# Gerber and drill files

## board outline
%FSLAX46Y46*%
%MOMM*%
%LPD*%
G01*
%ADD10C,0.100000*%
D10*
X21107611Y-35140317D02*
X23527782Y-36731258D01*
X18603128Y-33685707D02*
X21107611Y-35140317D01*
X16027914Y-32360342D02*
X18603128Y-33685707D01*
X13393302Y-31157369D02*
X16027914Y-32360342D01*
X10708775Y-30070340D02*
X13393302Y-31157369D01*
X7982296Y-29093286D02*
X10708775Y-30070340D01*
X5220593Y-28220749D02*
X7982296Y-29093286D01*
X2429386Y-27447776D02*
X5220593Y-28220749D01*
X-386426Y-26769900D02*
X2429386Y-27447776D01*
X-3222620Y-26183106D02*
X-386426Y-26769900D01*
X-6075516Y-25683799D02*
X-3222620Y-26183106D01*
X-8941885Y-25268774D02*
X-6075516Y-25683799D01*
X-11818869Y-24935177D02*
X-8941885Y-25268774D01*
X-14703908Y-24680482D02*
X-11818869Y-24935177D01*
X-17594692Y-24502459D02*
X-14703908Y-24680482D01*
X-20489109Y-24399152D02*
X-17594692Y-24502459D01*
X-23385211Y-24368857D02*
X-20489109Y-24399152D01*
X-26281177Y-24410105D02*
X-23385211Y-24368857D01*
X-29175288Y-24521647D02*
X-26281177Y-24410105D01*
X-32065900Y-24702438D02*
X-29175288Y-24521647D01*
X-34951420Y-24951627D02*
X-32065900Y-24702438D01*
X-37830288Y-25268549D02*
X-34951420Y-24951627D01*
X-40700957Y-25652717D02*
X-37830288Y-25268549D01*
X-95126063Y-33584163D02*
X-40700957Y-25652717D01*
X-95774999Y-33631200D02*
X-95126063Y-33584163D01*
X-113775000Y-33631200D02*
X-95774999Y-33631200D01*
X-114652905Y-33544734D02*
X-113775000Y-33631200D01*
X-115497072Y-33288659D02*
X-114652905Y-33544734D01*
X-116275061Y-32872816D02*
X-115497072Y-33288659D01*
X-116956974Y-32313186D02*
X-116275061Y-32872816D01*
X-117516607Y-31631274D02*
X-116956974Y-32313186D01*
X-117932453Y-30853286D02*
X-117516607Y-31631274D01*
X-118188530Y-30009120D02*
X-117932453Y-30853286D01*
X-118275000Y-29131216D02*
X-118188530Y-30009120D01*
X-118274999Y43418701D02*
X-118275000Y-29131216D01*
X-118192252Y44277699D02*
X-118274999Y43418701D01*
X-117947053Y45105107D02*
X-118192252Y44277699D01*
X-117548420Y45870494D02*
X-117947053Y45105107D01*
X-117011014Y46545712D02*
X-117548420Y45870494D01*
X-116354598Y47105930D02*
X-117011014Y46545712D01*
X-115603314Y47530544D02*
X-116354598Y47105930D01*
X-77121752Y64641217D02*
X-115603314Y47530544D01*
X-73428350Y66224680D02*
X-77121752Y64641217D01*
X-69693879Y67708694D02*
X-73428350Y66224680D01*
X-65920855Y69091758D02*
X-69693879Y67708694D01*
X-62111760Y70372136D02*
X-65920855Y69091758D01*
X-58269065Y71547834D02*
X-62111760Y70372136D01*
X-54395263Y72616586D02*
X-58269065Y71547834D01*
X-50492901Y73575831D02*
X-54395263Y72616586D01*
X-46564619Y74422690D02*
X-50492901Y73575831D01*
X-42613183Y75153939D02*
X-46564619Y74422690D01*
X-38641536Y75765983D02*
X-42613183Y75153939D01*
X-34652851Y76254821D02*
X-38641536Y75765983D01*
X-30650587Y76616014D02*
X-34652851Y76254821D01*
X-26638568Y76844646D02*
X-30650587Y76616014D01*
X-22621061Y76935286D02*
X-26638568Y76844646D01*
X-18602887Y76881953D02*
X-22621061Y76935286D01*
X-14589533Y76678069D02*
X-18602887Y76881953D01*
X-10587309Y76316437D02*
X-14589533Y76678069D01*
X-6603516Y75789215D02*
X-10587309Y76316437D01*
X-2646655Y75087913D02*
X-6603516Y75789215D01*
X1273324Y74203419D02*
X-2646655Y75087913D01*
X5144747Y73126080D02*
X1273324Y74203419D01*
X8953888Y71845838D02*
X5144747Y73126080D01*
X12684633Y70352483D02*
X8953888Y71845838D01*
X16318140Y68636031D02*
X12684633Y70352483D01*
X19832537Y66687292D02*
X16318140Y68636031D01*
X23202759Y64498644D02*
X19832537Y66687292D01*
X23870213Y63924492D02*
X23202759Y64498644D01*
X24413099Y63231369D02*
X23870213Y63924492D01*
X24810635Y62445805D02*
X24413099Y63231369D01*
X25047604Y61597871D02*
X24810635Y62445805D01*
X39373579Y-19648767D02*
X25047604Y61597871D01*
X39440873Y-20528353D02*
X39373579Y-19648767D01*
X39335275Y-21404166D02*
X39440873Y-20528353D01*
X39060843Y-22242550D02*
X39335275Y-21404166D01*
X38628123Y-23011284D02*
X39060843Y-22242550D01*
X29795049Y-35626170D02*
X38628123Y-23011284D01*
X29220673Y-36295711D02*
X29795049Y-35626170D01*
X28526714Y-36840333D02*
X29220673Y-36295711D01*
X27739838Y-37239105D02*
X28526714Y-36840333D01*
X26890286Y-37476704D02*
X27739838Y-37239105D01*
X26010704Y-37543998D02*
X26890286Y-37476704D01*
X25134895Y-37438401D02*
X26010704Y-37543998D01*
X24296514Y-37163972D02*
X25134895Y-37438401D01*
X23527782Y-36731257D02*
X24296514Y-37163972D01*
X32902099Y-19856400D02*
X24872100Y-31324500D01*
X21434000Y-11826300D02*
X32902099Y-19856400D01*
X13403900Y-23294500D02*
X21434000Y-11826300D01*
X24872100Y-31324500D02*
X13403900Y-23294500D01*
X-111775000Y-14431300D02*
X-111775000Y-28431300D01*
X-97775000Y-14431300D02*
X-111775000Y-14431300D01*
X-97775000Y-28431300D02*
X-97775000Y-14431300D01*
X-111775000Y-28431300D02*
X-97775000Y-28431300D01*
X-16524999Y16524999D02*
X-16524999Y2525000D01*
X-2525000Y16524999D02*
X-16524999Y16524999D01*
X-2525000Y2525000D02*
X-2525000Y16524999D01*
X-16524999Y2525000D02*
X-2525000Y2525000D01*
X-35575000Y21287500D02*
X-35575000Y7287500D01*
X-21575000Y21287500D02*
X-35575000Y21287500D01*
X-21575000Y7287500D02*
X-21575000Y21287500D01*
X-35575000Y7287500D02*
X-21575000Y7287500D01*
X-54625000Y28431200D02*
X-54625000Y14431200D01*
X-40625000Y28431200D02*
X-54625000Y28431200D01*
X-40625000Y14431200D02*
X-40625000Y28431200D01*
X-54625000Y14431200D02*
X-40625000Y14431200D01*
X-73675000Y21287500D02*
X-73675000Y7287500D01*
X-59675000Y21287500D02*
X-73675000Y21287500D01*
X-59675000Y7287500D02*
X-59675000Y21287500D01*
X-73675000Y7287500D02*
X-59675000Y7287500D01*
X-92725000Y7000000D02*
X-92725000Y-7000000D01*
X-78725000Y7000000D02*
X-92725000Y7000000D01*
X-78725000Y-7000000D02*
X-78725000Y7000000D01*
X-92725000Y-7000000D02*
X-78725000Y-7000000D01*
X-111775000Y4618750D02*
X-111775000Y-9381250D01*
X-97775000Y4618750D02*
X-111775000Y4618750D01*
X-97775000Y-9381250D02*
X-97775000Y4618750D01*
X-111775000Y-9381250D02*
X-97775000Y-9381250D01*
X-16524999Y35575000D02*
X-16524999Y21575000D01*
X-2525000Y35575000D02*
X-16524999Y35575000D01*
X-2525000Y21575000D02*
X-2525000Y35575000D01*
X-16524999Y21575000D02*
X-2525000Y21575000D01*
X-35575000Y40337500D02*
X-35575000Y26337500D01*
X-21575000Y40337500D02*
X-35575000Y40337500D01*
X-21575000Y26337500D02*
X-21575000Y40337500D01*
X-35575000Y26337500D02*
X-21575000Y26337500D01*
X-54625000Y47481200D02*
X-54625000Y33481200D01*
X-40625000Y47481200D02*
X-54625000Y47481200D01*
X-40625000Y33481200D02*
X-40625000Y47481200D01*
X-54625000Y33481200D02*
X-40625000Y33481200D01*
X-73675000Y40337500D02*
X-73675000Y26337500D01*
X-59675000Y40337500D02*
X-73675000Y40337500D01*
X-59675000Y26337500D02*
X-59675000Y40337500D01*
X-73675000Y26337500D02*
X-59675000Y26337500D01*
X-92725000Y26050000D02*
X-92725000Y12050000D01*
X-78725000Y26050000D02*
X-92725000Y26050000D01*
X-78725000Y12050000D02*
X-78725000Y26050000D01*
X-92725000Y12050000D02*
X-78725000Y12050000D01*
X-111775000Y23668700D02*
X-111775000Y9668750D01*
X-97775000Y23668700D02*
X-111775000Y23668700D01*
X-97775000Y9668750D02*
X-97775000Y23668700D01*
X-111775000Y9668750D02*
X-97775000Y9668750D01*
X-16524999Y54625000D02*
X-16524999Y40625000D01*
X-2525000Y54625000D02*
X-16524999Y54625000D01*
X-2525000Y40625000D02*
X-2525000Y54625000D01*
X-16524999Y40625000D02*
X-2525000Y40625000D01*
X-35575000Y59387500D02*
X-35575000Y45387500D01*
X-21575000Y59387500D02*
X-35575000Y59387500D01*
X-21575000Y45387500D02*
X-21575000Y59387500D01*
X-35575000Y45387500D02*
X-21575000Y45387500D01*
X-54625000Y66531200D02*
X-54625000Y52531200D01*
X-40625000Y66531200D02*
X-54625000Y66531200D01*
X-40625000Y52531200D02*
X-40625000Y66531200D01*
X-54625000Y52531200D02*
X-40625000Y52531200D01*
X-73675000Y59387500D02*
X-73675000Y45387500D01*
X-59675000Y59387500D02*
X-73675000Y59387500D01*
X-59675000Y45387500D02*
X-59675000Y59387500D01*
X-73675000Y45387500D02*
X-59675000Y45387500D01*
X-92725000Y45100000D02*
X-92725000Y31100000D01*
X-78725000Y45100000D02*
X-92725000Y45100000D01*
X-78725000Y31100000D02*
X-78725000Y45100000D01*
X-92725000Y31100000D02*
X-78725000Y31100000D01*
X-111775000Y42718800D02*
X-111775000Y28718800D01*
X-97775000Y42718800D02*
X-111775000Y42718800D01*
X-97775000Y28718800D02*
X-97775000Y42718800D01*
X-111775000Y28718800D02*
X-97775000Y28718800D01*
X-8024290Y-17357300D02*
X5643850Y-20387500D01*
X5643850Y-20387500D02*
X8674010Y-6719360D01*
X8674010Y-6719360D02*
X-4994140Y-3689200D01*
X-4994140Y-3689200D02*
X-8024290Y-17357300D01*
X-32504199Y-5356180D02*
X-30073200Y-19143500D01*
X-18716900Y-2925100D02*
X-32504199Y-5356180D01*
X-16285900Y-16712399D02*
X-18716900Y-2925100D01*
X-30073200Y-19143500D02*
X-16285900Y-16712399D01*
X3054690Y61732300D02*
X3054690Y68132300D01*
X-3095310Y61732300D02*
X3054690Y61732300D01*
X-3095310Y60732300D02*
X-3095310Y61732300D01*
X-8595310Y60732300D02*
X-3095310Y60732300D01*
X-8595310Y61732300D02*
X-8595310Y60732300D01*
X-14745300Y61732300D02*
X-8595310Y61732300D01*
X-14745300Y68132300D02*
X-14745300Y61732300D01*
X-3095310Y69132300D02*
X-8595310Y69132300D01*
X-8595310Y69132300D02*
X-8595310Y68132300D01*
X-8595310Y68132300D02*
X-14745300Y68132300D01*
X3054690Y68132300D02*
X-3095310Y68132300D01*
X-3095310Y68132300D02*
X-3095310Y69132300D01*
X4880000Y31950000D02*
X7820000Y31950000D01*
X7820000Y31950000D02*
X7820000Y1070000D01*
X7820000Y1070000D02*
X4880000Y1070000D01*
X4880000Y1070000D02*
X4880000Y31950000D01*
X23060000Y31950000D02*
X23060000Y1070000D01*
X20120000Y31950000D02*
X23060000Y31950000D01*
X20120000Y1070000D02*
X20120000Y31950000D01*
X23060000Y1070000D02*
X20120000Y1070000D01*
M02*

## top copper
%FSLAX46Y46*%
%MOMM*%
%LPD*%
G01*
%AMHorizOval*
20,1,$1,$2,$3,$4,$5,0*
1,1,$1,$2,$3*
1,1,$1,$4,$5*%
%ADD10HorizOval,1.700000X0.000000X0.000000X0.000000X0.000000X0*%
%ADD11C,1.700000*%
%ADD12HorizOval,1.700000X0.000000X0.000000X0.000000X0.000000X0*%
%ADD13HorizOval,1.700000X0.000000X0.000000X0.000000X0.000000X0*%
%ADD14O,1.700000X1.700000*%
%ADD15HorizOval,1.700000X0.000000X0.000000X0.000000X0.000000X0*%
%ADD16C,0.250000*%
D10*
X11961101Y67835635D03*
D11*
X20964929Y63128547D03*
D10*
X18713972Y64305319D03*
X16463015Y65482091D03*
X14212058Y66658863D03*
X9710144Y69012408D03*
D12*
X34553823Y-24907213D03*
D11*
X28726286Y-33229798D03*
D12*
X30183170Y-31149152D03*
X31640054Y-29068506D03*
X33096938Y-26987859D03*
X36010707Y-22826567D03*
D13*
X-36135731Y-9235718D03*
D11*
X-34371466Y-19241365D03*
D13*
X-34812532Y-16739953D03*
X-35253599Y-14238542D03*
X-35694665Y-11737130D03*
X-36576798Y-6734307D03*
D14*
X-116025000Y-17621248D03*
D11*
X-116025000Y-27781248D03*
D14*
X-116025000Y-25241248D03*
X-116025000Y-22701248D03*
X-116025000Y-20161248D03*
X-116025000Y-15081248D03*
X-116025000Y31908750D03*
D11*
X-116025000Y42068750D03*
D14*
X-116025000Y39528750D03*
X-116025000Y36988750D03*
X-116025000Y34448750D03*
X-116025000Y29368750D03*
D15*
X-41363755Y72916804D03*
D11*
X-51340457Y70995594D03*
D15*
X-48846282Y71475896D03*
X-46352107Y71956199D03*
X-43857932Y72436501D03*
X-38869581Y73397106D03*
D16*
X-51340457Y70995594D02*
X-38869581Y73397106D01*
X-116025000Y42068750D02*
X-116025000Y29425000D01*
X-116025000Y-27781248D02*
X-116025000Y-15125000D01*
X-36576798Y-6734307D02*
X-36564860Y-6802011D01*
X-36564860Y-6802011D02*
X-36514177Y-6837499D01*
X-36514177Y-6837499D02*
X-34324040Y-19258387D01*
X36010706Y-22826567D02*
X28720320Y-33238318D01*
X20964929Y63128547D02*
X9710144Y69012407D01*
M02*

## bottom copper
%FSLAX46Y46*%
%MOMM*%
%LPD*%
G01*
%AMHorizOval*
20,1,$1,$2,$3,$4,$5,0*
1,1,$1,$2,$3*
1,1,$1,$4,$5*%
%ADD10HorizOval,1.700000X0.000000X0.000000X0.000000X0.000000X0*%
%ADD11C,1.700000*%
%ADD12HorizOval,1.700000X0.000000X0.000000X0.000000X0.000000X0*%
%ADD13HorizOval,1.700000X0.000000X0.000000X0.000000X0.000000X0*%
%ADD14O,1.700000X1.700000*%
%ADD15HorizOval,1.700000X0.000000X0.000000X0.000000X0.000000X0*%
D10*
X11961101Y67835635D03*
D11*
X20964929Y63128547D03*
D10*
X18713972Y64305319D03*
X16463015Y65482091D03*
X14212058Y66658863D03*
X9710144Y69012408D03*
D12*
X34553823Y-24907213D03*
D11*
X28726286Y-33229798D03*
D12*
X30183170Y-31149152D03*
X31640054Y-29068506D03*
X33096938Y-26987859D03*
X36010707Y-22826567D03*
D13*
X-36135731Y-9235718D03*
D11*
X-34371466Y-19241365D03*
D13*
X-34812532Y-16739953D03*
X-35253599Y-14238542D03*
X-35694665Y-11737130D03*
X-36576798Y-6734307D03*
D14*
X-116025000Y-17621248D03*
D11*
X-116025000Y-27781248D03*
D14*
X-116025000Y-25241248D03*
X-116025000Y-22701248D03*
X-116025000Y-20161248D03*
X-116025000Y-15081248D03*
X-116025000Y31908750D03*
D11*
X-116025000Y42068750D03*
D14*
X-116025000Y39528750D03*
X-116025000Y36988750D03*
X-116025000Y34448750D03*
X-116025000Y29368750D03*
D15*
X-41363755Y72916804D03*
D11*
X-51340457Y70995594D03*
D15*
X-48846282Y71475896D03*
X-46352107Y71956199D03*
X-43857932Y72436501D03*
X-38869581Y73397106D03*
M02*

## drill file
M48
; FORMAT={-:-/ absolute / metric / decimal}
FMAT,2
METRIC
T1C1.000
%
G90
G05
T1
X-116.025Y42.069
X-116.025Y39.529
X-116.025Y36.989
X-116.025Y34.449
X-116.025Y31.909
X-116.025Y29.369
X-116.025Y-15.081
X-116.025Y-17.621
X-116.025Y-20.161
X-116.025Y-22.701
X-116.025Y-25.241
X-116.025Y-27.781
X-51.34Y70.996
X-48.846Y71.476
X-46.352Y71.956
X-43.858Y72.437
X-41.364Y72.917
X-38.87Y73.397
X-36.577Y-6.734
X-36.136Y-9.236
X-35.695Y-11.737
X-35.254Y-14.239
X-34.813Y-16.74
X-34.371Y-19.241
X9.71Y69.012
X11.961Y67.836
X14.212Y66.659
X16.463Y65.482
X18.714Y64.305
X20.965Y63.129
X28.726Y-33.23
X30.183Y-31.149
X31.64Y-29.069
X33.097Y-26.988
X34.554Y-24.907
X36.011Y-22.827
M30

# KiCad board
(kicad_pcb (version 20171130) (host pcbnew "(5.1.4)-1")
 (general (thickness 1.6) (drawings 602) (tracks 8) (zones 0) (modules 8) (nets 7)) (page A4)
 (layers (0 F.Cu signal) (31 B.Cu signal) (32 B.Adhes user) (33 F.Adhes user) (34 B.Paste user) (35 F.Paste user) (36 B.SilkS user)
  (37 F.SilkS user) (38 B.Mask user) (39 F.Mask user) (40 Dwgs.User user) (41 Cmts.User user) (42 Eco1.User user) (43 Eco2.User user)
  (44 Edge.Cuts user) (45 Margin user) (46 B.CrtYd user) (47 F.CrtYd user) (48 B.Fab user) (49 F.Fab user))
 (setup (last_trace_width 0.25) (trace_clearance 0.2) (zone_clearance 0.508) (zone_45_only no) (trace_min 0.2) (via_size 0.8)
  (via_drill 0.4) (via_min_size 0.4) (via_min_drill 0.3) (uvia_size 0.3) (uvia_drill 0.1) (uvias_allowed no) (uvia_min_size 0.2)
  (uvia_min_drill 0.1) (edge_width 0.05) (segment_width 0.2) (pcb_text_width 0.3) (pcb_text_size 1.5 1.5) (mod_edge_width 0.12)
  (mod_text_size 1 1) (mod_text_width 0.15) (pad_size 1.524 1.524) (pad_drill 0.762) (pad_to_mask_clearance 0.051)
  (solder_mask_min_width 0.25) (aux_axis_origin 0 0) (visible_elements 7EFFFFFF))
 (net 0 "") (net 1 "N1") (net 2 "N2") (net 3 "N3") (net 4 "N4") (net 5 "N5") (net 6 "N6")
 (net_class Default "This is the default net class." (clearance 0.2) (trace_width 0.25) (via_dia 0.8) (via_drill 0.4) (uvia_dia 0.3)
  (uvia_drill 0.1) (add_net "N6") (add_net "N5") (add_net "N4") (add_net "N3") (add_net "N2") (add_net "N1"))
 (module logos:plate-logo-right (layer B.Cu) (at 13.97 -26.2255 180)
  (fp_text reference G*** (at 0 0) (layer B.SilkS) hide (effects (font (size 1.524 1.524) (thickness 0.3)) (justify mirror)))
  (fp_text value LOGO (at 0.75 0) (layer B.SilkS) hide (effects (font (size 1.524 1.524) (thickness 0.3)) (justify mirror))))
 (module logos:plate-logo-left (layer F.Cu) (at 13.97 -26.2255)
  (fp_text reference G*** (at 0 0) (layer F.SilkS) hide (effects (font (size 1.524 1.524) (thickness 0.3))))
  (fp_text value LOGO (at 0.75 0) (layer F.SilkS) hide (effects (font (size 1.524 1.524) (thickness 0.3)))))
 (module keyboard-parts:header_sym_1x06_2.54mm (layer F.Cu) (at 20.964929 -63.128547 242.4)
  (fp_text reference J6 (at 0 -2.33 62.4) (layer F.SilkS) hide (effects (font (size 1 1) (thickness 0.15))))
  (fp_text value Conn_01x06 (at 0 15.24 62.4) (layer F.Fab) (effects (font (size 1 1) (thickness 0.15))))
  (pad 5 thru_hole oval (at 0 10.16 242.4) (size 1.7 1.7) (drill 1) (layers *.Cu *.Mask) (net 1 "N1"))
  (pad 1 thru_hole circle (at 0 0 242.4) (size 1.7 1.7) (drill 1) (layers *.Cu *.Mask) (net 1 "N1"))
  (pad 2 thru_hole oval (at 0 2.54 242.4) (size 1.7 1.7) (drill 1) (layers *.Cu *.Mask) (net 1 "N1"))
  (pad 3 thru_hole oval (at 0 5.08 242.4) (size 1.7 1.7) (drill 1) (layers *.Cu *.Mask) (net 1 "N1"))
  (pad 4 thru_hole oval (at 0 7.62 242.4) (size 1.7 1.7) (drill 1) (layers *.Cu *.Mask) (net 1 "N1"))
  (pad 6 thru_hole oval (at -0.000001 12.7 242.4) (size 1.7 1.7) (drill 1) (layers *.Cu *.Mask) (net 1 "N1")))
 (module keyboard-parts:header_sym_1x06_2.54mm (layer F.Cu) (at 28.726286 33.229798 145)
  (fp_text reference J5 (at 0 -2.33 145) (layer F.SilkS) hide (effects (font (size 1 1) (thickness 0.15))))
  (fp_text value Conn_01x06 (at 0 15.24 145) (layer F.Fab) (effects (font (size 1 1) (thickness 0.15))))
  (pad 5 thru_hole oval (at 0 10.16 145) (size 1.7 1.7) (drill 1) (layers *.Cu *.Mask) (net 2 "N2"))
  (pad 1 thru_hole circle (at 0 0 145) (size 1.7 1.7) (drill 1) (layers *.Cu *.Mask) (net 2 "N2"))
  (pad 2 thru_hole oval (at 0 2.54 145) (size 1.7 1.7) (drill 1) (layers *.Cu *.Mask) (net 2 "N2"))
  (pad 3 thru_hole oval (at 0 5.08 145) (size 1.7 1.7) (drill 1) (layers *.Cu *.Mask) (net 2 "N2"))
  (pad 4 thru_hole oval (at 0.000001 7.62 145) (size 1.7 1.7) (drill 1) (layers *.Cu *.Mask) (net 2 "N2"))
  (pad 6 thru_hole oval (at 0 12.7 145) (size 1.7 1.7) (drill 1) (layers *.Cu *.Mask) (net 2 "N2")))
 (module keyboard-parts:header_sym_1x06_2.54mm (layer F.Cu) (at -34.371466 19.241365 190)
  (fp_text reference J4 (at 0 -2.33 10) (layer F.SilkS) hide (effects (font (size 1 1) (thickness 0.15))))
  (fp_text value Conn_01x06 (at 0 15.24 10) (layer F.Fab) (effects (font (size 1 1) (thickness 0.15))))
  (pad 5 thru_hole oval (at -0.000001 10.16 190) (size 1.7 1.7) (drill 1) (layers *.Cu *.Mask) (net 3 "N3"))
  (pad 1 thru_hole circle (at 0 0 190) (size 1.7 1.7) (drill 1) (layers *.Cu *.Mask) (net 3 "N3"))
  (pad 2 thru_hole oval (at 0 2.54 190) (size 1.7 1.7) (drill 1) (layers *.Cu *.Mask) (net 3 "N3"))
  (pad 3 thru_hole oval (at 0 5.08 190) (size 1.7 1.7) (drill 1) (layers *.Cu *.Mask) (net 3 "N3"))
  (pad 4 thru_hole oval (at 0 7.62 190) (size 1.7 1.7) (drill 1) (layers *.Cu *.Mask) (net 3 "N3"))
  (pad 6 thru_hole oval (at 0 12.7 190) (size 1.7 1.7) (drill 1) (layers *.Cu *.Mask) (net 3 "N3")))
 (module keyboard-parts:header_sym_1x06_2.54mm (layer F.Cu) (at -116.025 27.781248 180)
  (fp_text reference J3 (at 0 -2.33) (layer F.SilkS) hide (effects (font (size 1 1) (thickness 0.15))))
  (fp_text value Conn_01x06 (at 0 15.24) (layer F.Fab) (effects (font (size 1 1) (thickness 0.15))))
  (pad 5 thru_hole oval (at 0 10.16 180) (size 1.7 1.7) (drill 1) (layers *.Cu *.Mask) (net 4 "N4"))
  (pad 1 thru_hole circle (at 0 0 180) (size 1.7 1.7) (drill 1) (layers *.Cu *.Mask) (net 4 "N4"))
  (pad 2 thru_hole oval (at 0 2.54 180) (size 1.7 1.7) (drill 1) (layers *.Cu *.Mask) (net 4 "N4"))
  (pad 3 thru_hole oval (at 0 5.08 180) (size 1.7 1.7) (drill 1) (layers *.Cu *.Mask) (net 4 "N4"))
  (pad 4 thru_hole oval (at 0 7.62 180) (size 1.7 1.7) (drill 1) (layers *.Cu *.Mask) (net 4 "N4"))
  (pad 6 thru_hole oval (at 0 12.7 180) (size 1.7 1.7) (drill 1) (layers *.Cu *.Mask) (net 4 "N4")))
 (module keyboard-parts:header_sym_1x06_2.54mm (layer F.Cu) (at -116.025 -42.06875)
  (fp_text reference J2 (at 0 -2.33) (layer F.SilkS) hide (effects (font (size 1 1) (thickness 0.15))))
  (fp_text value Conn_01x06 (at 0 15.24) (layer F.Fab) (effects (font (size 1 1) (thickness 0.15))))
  (pad 5 thru_hole oval (at 0 10.16) (size 1.7 1.7) (drill 1) (layers *.Cu *.Mask) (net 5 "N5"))
  (pad 1 thru_hole circle (at 0 0) (size 1.7 1.7) (drill 1) (layers *.Cu *.Mask) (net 5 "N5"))
  (pad 2 thru_hole oval (at 0 2.54) (size 1.7 1.7) (drill 1) (layers *.Cu *.Mask) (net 5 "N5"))
  (pad 3 thru_hole oval (at 0 5.08) (size 1.7 1.7) (drill 1) (layers *.Cu *.Mask) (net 5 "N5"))
  (pad 4 thru_hole oval (at 0 7.62) (size 1.7 1.7) (drill 1) (layers *.Cu *.Mask) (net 5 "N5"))
  (pad 6 thru_hole oval (at 0 12.7) (size 1.7 1.7) (drill 1) (layers *.Cu *.Mask) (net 5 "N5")))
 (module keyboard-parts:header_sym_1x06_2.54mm (layer F.Cu) (at -51.340457 -70.995594 100.9)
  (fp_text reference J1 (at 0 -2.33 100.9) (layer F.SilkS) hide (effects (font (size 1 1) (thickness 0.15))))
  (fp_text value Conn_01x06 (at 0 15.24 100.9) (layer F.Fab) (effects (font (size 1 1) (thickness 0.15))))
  (pad 5 thru_hole oval (at 0 10.160001 100.9) (size 1.7 1.7) (drill 1) (layers *.Cu *.Mask) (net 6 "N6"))
  (pad 1 thru_hole circle (at 0 0 100.9) (size 1.7 1.7) (drill 1) (layers *.Cu *.Mask) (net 6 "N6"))
  (pad 2 thru_hole oval (at 0 2.54 100.9) (size 1.7 1.7) (drill 1) (layers *.Cu *.Mask) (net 6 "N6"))
  (pad 3 thru_hole oval (at 0 5.08 100.9) (size 1.7 1.7) (drill 1) (layers *.Cu *.Mask) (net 6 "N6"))
  (pad 4 thru_hole oval (at 0 7.62 100.9) (size 1.7 1.7) (drill 1) (layers *.Cu *.Mask) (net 6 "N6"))
  (pad 6 thru_hole oval (at 0 12.7 100.9) (size 1.7 1.7) (drill 1) (layers *.Cu *.Mask) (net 6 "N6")))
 (gr_line (start 21.107611 35.140317) (end 23.527782 36.731258) (layer Edge.Cuts) (width 0.1))
 (gr_line (start 18.603128 33.685707) (end 21.107611 35.140317) (layer Edge.Cuts) (width 0.1))
 (gr_line (start 16.027914 32.360342) (end 18.603128 33.685707) (layer Edge.Cuts) (width 0.1))
 (gr_line (start 13.393302 31.157369) (end 16.027914 32.360342) (layer Edge.Cuts) (width 0.1))
 (gr_line (start 10.708775 30.07034) (end 13.393302 31.157369) (layer Edge.Cuts) (width 0.1))
 (gr_line (start 7.982296 29.093286) (end 10.708775 30.07034) (layer Edge.Cuts) (width 0.1))
 (gr_line (start 5.220593 28.220749) (end 7.982296 29.093286) (layer Edge.Cuts) (width 0.1))
 (gr_line (start 2.429386 27.447776) (end 5.220593 28.220749) (layer Edge.Cuts) (width 0.1))
 (gr_line (start -0.386426 26.7699) (end 2.429386 27.447776) (layer Edge.Cuts) (width 0.1))
 (gr_line (start -3.22262 26.183106) (end -0.386426 26.7699) (layer Edge.Cuts) (width 0.1))
 (gr_line (start -6.075516 25.683799) (end -3.22262 26.183106) (layer Edge.Cuts) (width 0.1))
 (gr_line (start -8.941885 25.268774) (end -6.075516 25.683799) (layer Edge.Cuts) (width 0.1))
 (gr_line (start -11.818869 24.935177) (end -8.941885 25.268774) (layer Edge.Cuts) (width 0.1))
 (gr_line (start -14.703908 24.680482) (end -11.818869 24.935177) (layer Edge.Cuts) (width 0.1))
 (gr_line (start -17.594692 24.502459) (end -14.703908 24.680482) (layer Edge.Cuts) (width 0.1))
 (gr_line (start -20.489109 24.399152) (end -17.594692 24.502459) (layer Edge.Cuts) (width 0.1))
 (gr_line (start -23.385211 24.368857) (end -20.489109 24.399152) (layer Edge.Cuts) (width 0.1))
 (gr_line (start -26.281177 24.410105) (end -23.385211 24.368857) (layer Edge.Cuts) (width 0.1))
 (gr_line (start -29.175288 24.521647) (end -26.281177 24.410105) (layer Edge.Cuts) (width 0.1))
 (gr_line (start -32.0659 24.702438) (end -29.175288 24.521647) (layer Edge.Cuts) (width 0.1))
 (gr_line (start -34.95142 24.951627) (end -32.0659 24.702438) (layer Edge.Cuts) (width 0.1))
 (gr_line (start -37.830288 25.268549) (end -34.95142 24.951627) (layer Edge.Cuts) (width 0.1))
 (gr_line (start -40.700957 25.652717) (end -37.830288 25.268549) (layer Edge.Cuts) (width 0.1))
 (gr_line (start -95.126063 33.584163) (end -40.700957 25.652717) (layer Edge.Cuts) (width 0.1))
 (gr_line (start -95.774999 33.6312) (end -95.126063 33.584163) (layer Edge.Cuts) (width 0.1))
 (gr_line (start -113.775 33.6312) (end -95.774999 33.6312) (layer Edge.Cuts) (width 0.1))
 (gr_line (start -114.652905 33.544734) (end -113.775 33.6312) (layer Edge.Cuts) (width 0.1))
 (gr_line (start -115.497072 33.288659) (end -114.652905 33.544734) (layer Edge.Cuts) (width 0.1))
 (gr_line (start -116.275061 32.872816) (end -115.497072 33.288659) (layer Edge.Cuts) (width 0.1))
 (gr_line (start -116.956974 32.313186) (end -116.275061 32.872816) (layer Edge.Cuts) (width 0.1))
 (gr_line (start -117.516607 31.631274) (end -116.956974 32.313186) (layer Edge.Cuts) (width 0.1))
 (gr_line (start -117.932453 30.853286) (end -117.516607 31.631274) (layer Edge.Cuts) (width 0.1))
 (gr_line (start -118.18853 30.00912) (end -117.932453 30.853286) (layer Edge.Cuts) (width 0.1))
 (gr_line (start -118.275 29.131216) (end -118.18853 30.00912) (layer Edge.Cuts) (width 0.1))
 (gr_line (start -118.274999 -43.418701) (end -118.275 29.131216) (layer Edge.Cuts) (width 0.1))
 (gr_line (start -118.192252 -44.277699) (end -118.274999 -43.418701) (layer Edge.Cuts) (width 0.1))
 (gr_line (start -117.947053 -45.105107) (end -118.192252 -44.277699) (layer Edge.Cuts) (width 0.1))
 (gr_line (start -117.54842 -45.870494) (end -117.947053 -45.105107) (layer Edge.Cuts) (width 0.1))
 (gr_line (start -117.011014 -46.545712) (end -117.54842 -45.870494) (layer Edge.Cuts) (width 0.1))
 (gr_line (start -116.354598 -47.10593) (end -117.011014 -46.545712) (layer Edge.Cuts) (width 0.1))
 (gr_line (start -115.603314 -47.530544) (end -116.354598 -47.10593) (layer Edge.Cuts) (width 0.1))
 (gr_line (start -77.121752 -64.641217) (end -115.603314 -47.530544) (layer Edge.Cuts) (width 0.1))
 (gr_line (start -73.42835 -66.22468) (end -77.121752 -64.641217) (layer Edge.Cuts) (width 0.1))
 (gr_line (start -69.693879 -67.708694) (end -73.42835 -66.22468) (layer Edge.Cuts) (width 0.1))
 (gr_line (start -65.920855 -69.091758) (end -69.693879 -67.708694) (layer Edge.Cuts) (width 0.1))
 (gr_line (start -62.11176 -70.372136) (end -65.920855 -69.091758) (layer Edge.Cuts) (width 0.1))
 (gr_line (start -58.269065 -71.547834) (end -62.11176 -70.372136) (layer Edge.Cuts) (width 0.1))
 (gr_line (start -54.395263 -72.616586) (end -58.269065 -71.547834) (layer Edge.Cuts) (width 0.1))
 (gr_line (start -50.492901 -73.575831) (end -54.395263 -72.616586) (layer Edge.Cuts) (width 0.1))
 (gr_line (start -46.564619 -74.42269) (end -50.492901 -73.575831) (layer Edge.Cuts) (width 0.1))
 (gr_line (start -42.613183 -75.153939) (end -46.564619 -74.42269) (layer Edge.Cuts) (width 0.1))
 (gr_line (start -38.641536 -75.765983) (end -42.613183 -75.153939) (layer Edge.Cuts) (width 0.1))
 (gr_line (start -34.652851 -76.254821) (end -38.641536 -75.765983) (layer Edge.Cuts) (width 0.1))
 (gr_line (start -30.650587 -76.616014) (end -34.652851 -76.254821) (layer Edge.Cuts) (width 0.1))
 (gr_line (start -26.638568 -76.844646) (end -30.650587 -76.616014) (layer Edge.Cuts) (width 0.1))
 (gr_line (start -22.621061 -76.935286) (end -26.638568 -76.844646) (layer Edge.Cuts) (width 0.1))
 (gr_line (start -18.602887 -76.881953) (end -22.621061 -76.935286) (layer Edge.Cuts) (width 0.1))
 (gr_line (start -14.589533 -76.678069) (end -18.602887 -76.881953) (layer Edge.Cuts) (width 0.1))
 (gr_line (start -10.587309 -76.316437) (end -14.589533 -76.678069) (layer Edge.Cuts) (width 0.1))
 (gr_line (start -6.603516 -75.789215) (end -10.587309 -76.316437) (layer Edge.Cuts) (width 0.1))
 (gr_line (start -2.646655 -75.087913) (end -6.603516 -75.789215) (layer Edge.Cuts) (width 0.1))
 (gr_line (start 1.273324 -74.203419) (end -2.646655 -75.087913) (layer Edge.Cuts) (width 0.1))
 (gr_line (start 5.144747 -73.12608) (end 1.273324 -74.203419) (layer Edge.Cuts) (width 0.1))
 (gr_line (start 8.953888 -71.845838) (end 5.144747 -73.12608) (layer Edge.Cuts) (width 0.1))
 (gr_line (start 12.684633 -70.352483) (end 8.953888 -71.845838) (layer Edge.Cuts) (width 0.1))
 (gr_line (start 16.31814 -68.636031) (end 12.684633 -70.352483) (layer Edge.Cuts) (width 0.1))
 (gr_line (start 19.832537 -66.687292) (end 16.31814 -68.636031) (layer Edge.Cuts) (width 0.1))
 (gr_line (start 23.202759 -64.498644) (end 19.832537 -66.687292) (layer Edge.Cuts) (width 0.1))
 (gr_line (start 23.870213 -63.924492) (end 23.202759 -64.498644) (layer Edge.Cuts) (width 0.1))
 (gr_line (start 24.413099 -63.231369) (end 23.870213 -63.924492) (layer Edge.Cuts) (width 0.1))
 (gr_line (start 24.810635 -62.445805) (end 24.413099 -63.231369) (layer Edge.Cuts) (width 0.1))
 (gr_line (start 25.047604 -61.597871) (end 24.810635 -62.445805) (layer Edge.Cuts) (width 0.1))
 (gr_line (start 39.373579 19.648767) (end 25.047604 -61.597871) (layer Edge.Cuts) (width 0.1))
 (gr_line (start 39.440873 20.528353) (end 39.373579 19.648767) (layer Edge.Cuts) (width 0.1))
 (gr_line (start 39.335275 21.404166) (end 39.440873 20.528353) (layer Edge.Cuts) (width 0.1))
 (gr_line (start 39.060843 22.24255) (end 39.335275 21.404166) (layer Edge.Cuts) (width 0.1))
 (gr_line (start 38.628123 23.011284) (end 39.060843 22.24255) (layer Edge.Cuts) (width 0.1))
 (gr_line (start 29.795049 35.62617) (end 38.628123 23.011284) (layer Edge.Cuts) (width 0.1))
 (gr_line (start 29.220673 36.295711) (end 29.795049 35.62617) (layer Edge.Cuts) (width 0.1))
 (gr_line (start 28.526714 36.840333) (end 29.220673 36.295711) (layer Edge.Cuts) (width 0.1))
 (gr_line (start 27.739838 37.239105) (end 28.526714 36.840333) (layer Edge.Cuts) (width 0.1))
 (gr_line (start 26.890286 37.476704) (end 27.739838 37.239105) (layer Edge.Cuts) (width 0.1))
 (gr_line (start 26.010704 37.543998) (end 26.890286 37.476704) (layer Edge.Cuts) (width 0.1))
 (gr_line (start 25.134895 37.438401) (end 26.010704 37.543998) (layer Edge.Cuts) (width 0.1))
 (gr_line (start 24.296514 37.163972) (end 25.134895 37.438401) (layer Edge.Cuts) (width 0.1))
 (gr_line (start 23.527782 36.731257) (end 24.296514 37.163972) (layer Edge.Cuts) (width 0.1))
 (gr_line (start 32.902099 19.8564) (end 24.8721 31.3245) (layer Edge.Cuts) (width 0.1))
 (gr_line (start 21.434 11.8263) (end 32.902099 19.8564) (layer Edge.Cuts) (width 0.1))
 (gr_line (start 13.4039 23.2945) (end 21.434 11.8263) (layer Edge.Cuts) (width 0.1))
 (gr_line (start 24.8721 31.3245) (end 13.4039 23.2945) (layer Edge.Cuts) (width 0.1))
 (gr_line (start -111.775 14.4313) (end -111.775 28.4313) (layer Edge.Cuts) (width 0.1))
 (gr_line (start -97.775 14.4313) (end -111.775 14.4313) (layer Edge.Cuts) (width 0.1))
 (gr_line (start -97.775 28.4313) (end -97.775 14.4313) (layer Edge.Cuts) (width 0.1))
 (gr_line (start -111.775 28.4313) (end -97.775 28.4313) (layer Edge.Cuts) (width 0.1))
 (gr_line (start -16.524999 -16.524999) (end -16.524999 -2.525) (layer Edge.Cuts) (width 0.1))
 (gr_line (start -2.525 -16.524999) (end -16.524999 -16.524999) (layer Edge.Cuts) (width 0.1))
 (gr_line (start -2.525 -2.525) (end -2.525 -16.524999) (layer Edge.Cuts) (width 0.1))
 (gr_line (start -16.524999 -2.525) (end -2.525 -2.525) (layer Edge.Cuts) (width 0.1))
 (gr_line (start -35.575 -21.2875) (end -35.575 -7.2875) (layer Edge.Cuts) (width 0.1))
 (gr_line (start -21.575 -21.2875) (end -35.575 -21.2875) (layer Edge.Cuts) (width 0.1))
 (gr_line (start -21.575 -7.2875) (end -21.575 -21.2875) (layer Edge.Cuts) (width 0.1))
 (gr_line (start -35.575 -7.2875) (end -21.575 -7.2875) (layer Edge.Cuts) (width 0.1))
 (gr_line (start -54.625 -28.4312) (end -54.625 -14.4312) (layer Edge.Cuts) (width 0.1))
 (gr_line (start -40.625 -28.4312) (end -54.625 -28.4312) (layer Edge.Cuts) (width 0.1))
 (gr_line (start -40.625 -14.4312) (end -40.625 -28.4312) (layer Edge.Cuts) (width 0.1))
 (gr_line (start -54.625 -14.4312) (end -40.625 -14.4312) (layer Edge.Cuts) (width 0.1))
 (gr_line (start -73.675 -21.2875) (end -73.675 -7.2875) (layer Edge.Cuts) (width 0.1))
 (gr_line (start -59.675 -21.2875) (end -73.675 -21.2875) (layer Edge.Cuts) (width 0.1))
 (gr_line (start -59.675 -7.2875) (end -59.675 -21.2875) (layer Edge.Cuts) (width 0.1))
 (gr_line (start -73.675 -7.2875) (end -59.675 -7.2875) (layer Edge.Cuts) (width 0.1))
 (gr_line (start -92.725 -7) (end -92.725 7) (layer Edge.Cuts) (width 0.1))
 (gr_line (start -78.725 -7) (end -92.725 -7) (layer Edge.Cuts) (width 0.1))
 (gr_line (start -78.725 7) (end -78.725 -7) (layer Edge.Cuts) (width 0.1))
 (gr_line (start -92.725 7) (end -78.725 7) (layer Edge.Cuts) (width 0.1))
 (gr_line (start -111.775 -4.61875) (end -111.775 9.38125) (layer Edge.Cuts) (width 0.1))
 (gr_line (start -97.775 -4.61875) (end -111.775 -4.61875) (layer Edge.Cuts) (width 0.1))
 (gr_line (start -97.775 9.38125) (end -97.775 -4.61875) (layer Edge.Cuts) (width 0.1))
 (gr_line (start -111.775 9.38125) (end -97.775 9.38125) (layer Edge.Cuts) (width 0.1))
 (gr_line (start -16.524999 -35.575) (end -16.524999 -21.575) (layer Edge.Cuts) (width 0.1))
 (gr_line (start -2.525 -35.575) (end -16.524999 -35.575) (layer Edge.Cuts) (width 0.1))
 (gr_line (start -2.525 -21.575) (end -2.525 -35.575) (layer Edge.Cuts) (width 0.1))
 (gr_line (start -16.524999 -21.575) (end -2.525 -21.575) (layer Edge.Cuts) (width 0.1))
 (gr_line (start -35.575 -40.3375) (end -35.575 -26.3375) (layer Edge.Cuts) (width 0.1))
 (gr_line (start -21.575 -40.3375) (end -35.575 -40.3375) (layer Edge.Cuts) (width 0.1))
 (gr_line (start -21.575 -26.3375) (end -21.575 -40.3375) (layer Edge.Cuts) (width 0.1))
 (gr_line (start -35.575 -26.3375) (end -21.575 -26.3375) (layer Edge.Cuts) (width 0.1))
 (gr_line (start -54.625 -47.4812) (end -54.625 -33.4812) (layer Edge.Cuts) (width 0.1))
 (gr_line (start -40.625 -47.4812) (end -54.625 -47.4812) (layer Edge.Cuts) (width 0.1))
 (gr_line (start -40.625 -33.4812) (end -40.625 -47.4812) (layer Edge.Cuts) (width 0.1))
 (gr_line (start -54.625 -33.4812) (end -40.625 -33.4812) (layer Edge.Cuts) (width 0.1))
 (gr_line (start -73.675 -40.3375) (end -73.675 -26.3375) (layer Edge.Cuts) (width 0.1))
 (gr_line (start -59.675 -40.3375) (end -73.675 -40.3375) (layer Edge.Cuts) (width 0.1))
 (gr_line (start -59.675 -26.3375) (end -59.675 -40.3375) (layer Edge.Cuts) (width 0.1))
 (gr_line (start -73.675 -26.3375) (end -59.675 -26.3375) (layer Edge.Cuts) (width 0.1))
 (gr_line (start -92.725 -26.05) (end -92.725 -12.05) (layer Edge.Cuts) (width 0.1))
 (gr_line (start -78.725 -26.05) (end -92.725 -26.05) (layer Edge.Cuts) (width 0.1))
 (gr_line (start -78.725 -12.05) (end -78.725 -26.05) (layer Edge.Cuts) (width 0.1))
 (gr_line (start -92.725 -12.05) (end -78.725 -12.05) (layer Edge.Cuts) (width 0.1))
 (gr_line (start -111.775 -23.6687) (end -111.775 -9.66875) (layer Edge.Cuts) (width 0.1))
 (gr_line (start -97.775 -23.6687) (end -111.775 -23.6687) (layer Edge.Cuts) (width 0.1))
 (gr_line (start -97.775 -9.66875) (end -97.775 -23.6687) (layer Edge.Cuts) (width 0.1))
 (gr_line (start -111.775 -9.66875) (end -97.775 -9.66875) (layer Edge.Cuts) (width 0.1))
 (gr_line (start -16.524999 -54.625) (end -16.524999 -40.625) (layer Edge.Cuts) (width 0.1))
 (gr_line (start -2.525 -54.625) (end -16.524999 -54.625) (layer Edge.Cuts) (width 0.1))
 (gr_line (start -2.525 -40.625) (end -2.525 -54.625) (layer Edge.Cuts) (width 0.1))
 (gr_line (start -16.524999 -40.625) (end -2.525 -40.625) (layer Edge.Cuts) (width 0.1))
 (gr_line (start -35.575 -59.3875) (end -35.575 -45.3875) (layer Edge.Cuts) (width 0.1))
 (gr_line (start -21.575 -59.3875) (end -35.575 -59.3875) (layer Edge.Cuts) (width 0.1))
 (gr_line (start -21.575 -45.3875) (end -21.575 -59.3875) (layer Edge.Cuts) (width 0.1))
 (gr_line (start -35.575 -45.3875) (end -21.575 -45.3875) (layer Edge.Cuts) (width 0.1))
 (gr_line (start -54.625 -66.5312) (end -54.625 -52.5312) (layer Edge.Cuts) (width 0.1))
 (gr_line (start -40.625 -66.5312) (end -54.625 -66.5312) (layer Edge.Cuts) (width 0.1))
 (gr_line (start -40.625 -52.5312) (end -40.625 -66.5312) (layer Edge.Cuts) (width 0.1))
 (gr_line (start -54.625 -52.5312) (end -40.625 -52.5312) (layer Edge.Cuts) (width 0.1))
 (gr_line (start -73.675 -59.3875) (end -73.675 -45.3875) (layer Edge.Cuts) (width 0.1))
 (gr_line (start -59.675 -59.3875) (end -73.675 -59.3875) (layer Edge.Cuts) (width 0.1))
 (gr_line (start -59.675 -45.3875) (end -59.675 -59.3875) (layer Edge.Cuts) (width 0.1))
 (gr_line (start -73.675 -45.3875) (end -59.675 -45.3875) (layer Edge.Cuts) (width 0.1))
 (gr_line (start -92.725 -45.1) (end -92.725 -31.1) (layer Edge.Cuts) (width 0.1))
 (gr_line (start -78.725 -45.1) (end -92.725 -45.1) (layer Edge.Cuts) (width 0.1))
 (gr_line (start -78.725 -31.1) (end -78.725 -45.1) (layer Edge.Cuts) (width 0.1))
 (gr_line (start -92.725 -31.1) (end -78.725 -31.1) (layer Edge.Cuts) (width 0.1))
 (gr_line (start -111.775 -42.7188) (end -111.775 -28.7188) (layer Edge.Cuts) (width 0.1))
 (gr_line (start -97.775 -42.7188) (end -111.775 -42.7188) (layer Edge.Cuts) (width 0.1))
 (gr_line (start -97.775 -28.7188) (end -97.775 -42.7188) (layer Edge.Cuts) (width 0.1))
 (gr_line (start -111.775 -28.7188) (end -97.775 -28.7188) (layer Edge.Cuts) (width 0.1))
 (gr_line (start -8.02429 17.3573) (end 5.64385 20.3875) (layer Edge.Cuts) (width 0.1))
 (gr_line (start 5.64385 20.3875) (end 8.67401 6.71936) (layer Edge.Cuts) (width 0.1))
 (gr_line (start 8.67401 6.71936) (end -4.99414 3.6892) (layer Edge.Cuts) (width 0.1))
 (gr_line (start -4.99414 3.6892) (end -8.02429 17.3573) (layer Edge.Cuts) (width 0.1))
 (gr_line (start -32.504199 5.35618) (end -30.0732 19.1435) (layer Edge.Cuts) (width 0.1))
 (gr_line (start -18.7169 2.9251) (end -32.504199 5.35618) (layer Edge.Cuts) (width 0.1))
 (gr_line (start -16.2859 16.712399) (end -18.7169 2.9251) (layer Edge.Cuts) (width 0.1))
 (gr_line (start -30.0732 19.1435) (end -16.2859 16.712399) (layer Edge.Cuts) (width 0.1))
 (gr_line (start 3.05469 -61.7323) (end 3.05469 -68.1323) (layer Edge.Cuts) (width 0.1))
 (gr_line (start -3.09531 -61.7323) (end 3.05469 -61.7323) (layer Edge.Cuts) (width 0.1))
 (gr_line (start -3.09531 -60.7323) (end -3.09531 -61.7323) (layer Edge.Cuts) (width 0.1))
 (gr_line (start -8.59531 -60.7323) (end -3.09531 -60.7323) (layer Edge.Cuts) (width 0.1))
 (gr_line (start -8.59531 -61.7323) (end -8.59531 -60.7323) (layer Edge.Cuts) (width 0.1))
 (gr_line (start -14.7453 -61.7323) (end -8.59531 -61.7323) (layer Edge.Cuts) (width 0.1))
 (gr_line (start -14.7453 -68.1323) (end -14.7453 -61.7323) (layer Edge.Cuts) (width 0.1))
 (gr_line (start -3.09531 -69.1323) (end -8.59531 -69.1323) (layer Edge.Cuts) (width 0.1))
 (gr_line (start -8.59531 -69.1323) (end -8.59531 -68.1323) (layer Edge.Cuts) (width 0.1))
 (gr_line (start -8.59531 -68.1323) (end -14.7453 -68.1323) (layer Edge.Cuts) (width 0.1))
 (gr_line (start 3.05469 -68.1323) (end -3.09531 -68.1323) (layer Edge.Cuts) (width 0.1))
 (gr_line (start -3.09531 -68.1323) (end -3.09531 -69.1323) (layer Edge.Cuts) (width 0.1))
 (gr_line (start 4.88 -31.95) (end 7.82 -31.95) (layer Edge.Cuts) (width 0.1))
 (gr_line (start 7.82 -31.95) (end 7.82 -1.07) (layer Edge.Cuts) (width 0.1))
 (gr_line (start 7.82 -1.07) (end 4.88 -1.07) (layer Edge.Cuts) (width 0.1))
 (gr_line (start 4.88 -1.07) (end 4.88 -31.95) (layer Edge.Cuts) (width 0.1))
 (gr_line (start 23.06 -31.95) (end 23.06 -1.07) (layer Edge.Cuts) (width 0.1))
 (gr_line (start 20.12 -31.95) (end 23.06 -31.95) (layer Edge.Cuts) (width 0.1))
 (gr_line (start 20.12 -1.07) (end 20.12 -31.95) (layer Edge.Cuts) (width 0.1))
 (gr_line (start 23.06 -1.07) (end 20.12 -1.07) (layer Edge.Cuts) (width 0.1))
 (segment (start -51.340457 -70.995594) (end -38.869581 -73.397106) (width 0.25) (layer F.Cu) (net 6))
 (segment (start -116.025 -42.06875) (end -116.025 -29.425) (width 0.25) (layer F.Cu) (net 5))
 (segment (start -116.025 27.781248) (end -116.025 15.125) (width 0.25) (layer F.Cu) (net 4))
 (segment (start -36.576798 6.734307) (end -36.56486 6.802011) (width 0.25) (layer F.Cu) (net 3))
 (segment (start -36.56486 6.802011) (end -36.514177 6.837499) (width 0.25) (layer F.Cu) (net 3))
 (segment (start -36.514177 6.837499) (end -34.32404 19.258387) (width 0.25) (layer F.Cu) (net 3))
 (segment (start 36.010706 22.826567) (end 28.72032 33.238318) (width 0.25) (layer F.Cu) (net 2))
 (segment (start 20.964929 -63.128547) (end 9.710144 -69.012407) (width 0.25) (layer F.Cu) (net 1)))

